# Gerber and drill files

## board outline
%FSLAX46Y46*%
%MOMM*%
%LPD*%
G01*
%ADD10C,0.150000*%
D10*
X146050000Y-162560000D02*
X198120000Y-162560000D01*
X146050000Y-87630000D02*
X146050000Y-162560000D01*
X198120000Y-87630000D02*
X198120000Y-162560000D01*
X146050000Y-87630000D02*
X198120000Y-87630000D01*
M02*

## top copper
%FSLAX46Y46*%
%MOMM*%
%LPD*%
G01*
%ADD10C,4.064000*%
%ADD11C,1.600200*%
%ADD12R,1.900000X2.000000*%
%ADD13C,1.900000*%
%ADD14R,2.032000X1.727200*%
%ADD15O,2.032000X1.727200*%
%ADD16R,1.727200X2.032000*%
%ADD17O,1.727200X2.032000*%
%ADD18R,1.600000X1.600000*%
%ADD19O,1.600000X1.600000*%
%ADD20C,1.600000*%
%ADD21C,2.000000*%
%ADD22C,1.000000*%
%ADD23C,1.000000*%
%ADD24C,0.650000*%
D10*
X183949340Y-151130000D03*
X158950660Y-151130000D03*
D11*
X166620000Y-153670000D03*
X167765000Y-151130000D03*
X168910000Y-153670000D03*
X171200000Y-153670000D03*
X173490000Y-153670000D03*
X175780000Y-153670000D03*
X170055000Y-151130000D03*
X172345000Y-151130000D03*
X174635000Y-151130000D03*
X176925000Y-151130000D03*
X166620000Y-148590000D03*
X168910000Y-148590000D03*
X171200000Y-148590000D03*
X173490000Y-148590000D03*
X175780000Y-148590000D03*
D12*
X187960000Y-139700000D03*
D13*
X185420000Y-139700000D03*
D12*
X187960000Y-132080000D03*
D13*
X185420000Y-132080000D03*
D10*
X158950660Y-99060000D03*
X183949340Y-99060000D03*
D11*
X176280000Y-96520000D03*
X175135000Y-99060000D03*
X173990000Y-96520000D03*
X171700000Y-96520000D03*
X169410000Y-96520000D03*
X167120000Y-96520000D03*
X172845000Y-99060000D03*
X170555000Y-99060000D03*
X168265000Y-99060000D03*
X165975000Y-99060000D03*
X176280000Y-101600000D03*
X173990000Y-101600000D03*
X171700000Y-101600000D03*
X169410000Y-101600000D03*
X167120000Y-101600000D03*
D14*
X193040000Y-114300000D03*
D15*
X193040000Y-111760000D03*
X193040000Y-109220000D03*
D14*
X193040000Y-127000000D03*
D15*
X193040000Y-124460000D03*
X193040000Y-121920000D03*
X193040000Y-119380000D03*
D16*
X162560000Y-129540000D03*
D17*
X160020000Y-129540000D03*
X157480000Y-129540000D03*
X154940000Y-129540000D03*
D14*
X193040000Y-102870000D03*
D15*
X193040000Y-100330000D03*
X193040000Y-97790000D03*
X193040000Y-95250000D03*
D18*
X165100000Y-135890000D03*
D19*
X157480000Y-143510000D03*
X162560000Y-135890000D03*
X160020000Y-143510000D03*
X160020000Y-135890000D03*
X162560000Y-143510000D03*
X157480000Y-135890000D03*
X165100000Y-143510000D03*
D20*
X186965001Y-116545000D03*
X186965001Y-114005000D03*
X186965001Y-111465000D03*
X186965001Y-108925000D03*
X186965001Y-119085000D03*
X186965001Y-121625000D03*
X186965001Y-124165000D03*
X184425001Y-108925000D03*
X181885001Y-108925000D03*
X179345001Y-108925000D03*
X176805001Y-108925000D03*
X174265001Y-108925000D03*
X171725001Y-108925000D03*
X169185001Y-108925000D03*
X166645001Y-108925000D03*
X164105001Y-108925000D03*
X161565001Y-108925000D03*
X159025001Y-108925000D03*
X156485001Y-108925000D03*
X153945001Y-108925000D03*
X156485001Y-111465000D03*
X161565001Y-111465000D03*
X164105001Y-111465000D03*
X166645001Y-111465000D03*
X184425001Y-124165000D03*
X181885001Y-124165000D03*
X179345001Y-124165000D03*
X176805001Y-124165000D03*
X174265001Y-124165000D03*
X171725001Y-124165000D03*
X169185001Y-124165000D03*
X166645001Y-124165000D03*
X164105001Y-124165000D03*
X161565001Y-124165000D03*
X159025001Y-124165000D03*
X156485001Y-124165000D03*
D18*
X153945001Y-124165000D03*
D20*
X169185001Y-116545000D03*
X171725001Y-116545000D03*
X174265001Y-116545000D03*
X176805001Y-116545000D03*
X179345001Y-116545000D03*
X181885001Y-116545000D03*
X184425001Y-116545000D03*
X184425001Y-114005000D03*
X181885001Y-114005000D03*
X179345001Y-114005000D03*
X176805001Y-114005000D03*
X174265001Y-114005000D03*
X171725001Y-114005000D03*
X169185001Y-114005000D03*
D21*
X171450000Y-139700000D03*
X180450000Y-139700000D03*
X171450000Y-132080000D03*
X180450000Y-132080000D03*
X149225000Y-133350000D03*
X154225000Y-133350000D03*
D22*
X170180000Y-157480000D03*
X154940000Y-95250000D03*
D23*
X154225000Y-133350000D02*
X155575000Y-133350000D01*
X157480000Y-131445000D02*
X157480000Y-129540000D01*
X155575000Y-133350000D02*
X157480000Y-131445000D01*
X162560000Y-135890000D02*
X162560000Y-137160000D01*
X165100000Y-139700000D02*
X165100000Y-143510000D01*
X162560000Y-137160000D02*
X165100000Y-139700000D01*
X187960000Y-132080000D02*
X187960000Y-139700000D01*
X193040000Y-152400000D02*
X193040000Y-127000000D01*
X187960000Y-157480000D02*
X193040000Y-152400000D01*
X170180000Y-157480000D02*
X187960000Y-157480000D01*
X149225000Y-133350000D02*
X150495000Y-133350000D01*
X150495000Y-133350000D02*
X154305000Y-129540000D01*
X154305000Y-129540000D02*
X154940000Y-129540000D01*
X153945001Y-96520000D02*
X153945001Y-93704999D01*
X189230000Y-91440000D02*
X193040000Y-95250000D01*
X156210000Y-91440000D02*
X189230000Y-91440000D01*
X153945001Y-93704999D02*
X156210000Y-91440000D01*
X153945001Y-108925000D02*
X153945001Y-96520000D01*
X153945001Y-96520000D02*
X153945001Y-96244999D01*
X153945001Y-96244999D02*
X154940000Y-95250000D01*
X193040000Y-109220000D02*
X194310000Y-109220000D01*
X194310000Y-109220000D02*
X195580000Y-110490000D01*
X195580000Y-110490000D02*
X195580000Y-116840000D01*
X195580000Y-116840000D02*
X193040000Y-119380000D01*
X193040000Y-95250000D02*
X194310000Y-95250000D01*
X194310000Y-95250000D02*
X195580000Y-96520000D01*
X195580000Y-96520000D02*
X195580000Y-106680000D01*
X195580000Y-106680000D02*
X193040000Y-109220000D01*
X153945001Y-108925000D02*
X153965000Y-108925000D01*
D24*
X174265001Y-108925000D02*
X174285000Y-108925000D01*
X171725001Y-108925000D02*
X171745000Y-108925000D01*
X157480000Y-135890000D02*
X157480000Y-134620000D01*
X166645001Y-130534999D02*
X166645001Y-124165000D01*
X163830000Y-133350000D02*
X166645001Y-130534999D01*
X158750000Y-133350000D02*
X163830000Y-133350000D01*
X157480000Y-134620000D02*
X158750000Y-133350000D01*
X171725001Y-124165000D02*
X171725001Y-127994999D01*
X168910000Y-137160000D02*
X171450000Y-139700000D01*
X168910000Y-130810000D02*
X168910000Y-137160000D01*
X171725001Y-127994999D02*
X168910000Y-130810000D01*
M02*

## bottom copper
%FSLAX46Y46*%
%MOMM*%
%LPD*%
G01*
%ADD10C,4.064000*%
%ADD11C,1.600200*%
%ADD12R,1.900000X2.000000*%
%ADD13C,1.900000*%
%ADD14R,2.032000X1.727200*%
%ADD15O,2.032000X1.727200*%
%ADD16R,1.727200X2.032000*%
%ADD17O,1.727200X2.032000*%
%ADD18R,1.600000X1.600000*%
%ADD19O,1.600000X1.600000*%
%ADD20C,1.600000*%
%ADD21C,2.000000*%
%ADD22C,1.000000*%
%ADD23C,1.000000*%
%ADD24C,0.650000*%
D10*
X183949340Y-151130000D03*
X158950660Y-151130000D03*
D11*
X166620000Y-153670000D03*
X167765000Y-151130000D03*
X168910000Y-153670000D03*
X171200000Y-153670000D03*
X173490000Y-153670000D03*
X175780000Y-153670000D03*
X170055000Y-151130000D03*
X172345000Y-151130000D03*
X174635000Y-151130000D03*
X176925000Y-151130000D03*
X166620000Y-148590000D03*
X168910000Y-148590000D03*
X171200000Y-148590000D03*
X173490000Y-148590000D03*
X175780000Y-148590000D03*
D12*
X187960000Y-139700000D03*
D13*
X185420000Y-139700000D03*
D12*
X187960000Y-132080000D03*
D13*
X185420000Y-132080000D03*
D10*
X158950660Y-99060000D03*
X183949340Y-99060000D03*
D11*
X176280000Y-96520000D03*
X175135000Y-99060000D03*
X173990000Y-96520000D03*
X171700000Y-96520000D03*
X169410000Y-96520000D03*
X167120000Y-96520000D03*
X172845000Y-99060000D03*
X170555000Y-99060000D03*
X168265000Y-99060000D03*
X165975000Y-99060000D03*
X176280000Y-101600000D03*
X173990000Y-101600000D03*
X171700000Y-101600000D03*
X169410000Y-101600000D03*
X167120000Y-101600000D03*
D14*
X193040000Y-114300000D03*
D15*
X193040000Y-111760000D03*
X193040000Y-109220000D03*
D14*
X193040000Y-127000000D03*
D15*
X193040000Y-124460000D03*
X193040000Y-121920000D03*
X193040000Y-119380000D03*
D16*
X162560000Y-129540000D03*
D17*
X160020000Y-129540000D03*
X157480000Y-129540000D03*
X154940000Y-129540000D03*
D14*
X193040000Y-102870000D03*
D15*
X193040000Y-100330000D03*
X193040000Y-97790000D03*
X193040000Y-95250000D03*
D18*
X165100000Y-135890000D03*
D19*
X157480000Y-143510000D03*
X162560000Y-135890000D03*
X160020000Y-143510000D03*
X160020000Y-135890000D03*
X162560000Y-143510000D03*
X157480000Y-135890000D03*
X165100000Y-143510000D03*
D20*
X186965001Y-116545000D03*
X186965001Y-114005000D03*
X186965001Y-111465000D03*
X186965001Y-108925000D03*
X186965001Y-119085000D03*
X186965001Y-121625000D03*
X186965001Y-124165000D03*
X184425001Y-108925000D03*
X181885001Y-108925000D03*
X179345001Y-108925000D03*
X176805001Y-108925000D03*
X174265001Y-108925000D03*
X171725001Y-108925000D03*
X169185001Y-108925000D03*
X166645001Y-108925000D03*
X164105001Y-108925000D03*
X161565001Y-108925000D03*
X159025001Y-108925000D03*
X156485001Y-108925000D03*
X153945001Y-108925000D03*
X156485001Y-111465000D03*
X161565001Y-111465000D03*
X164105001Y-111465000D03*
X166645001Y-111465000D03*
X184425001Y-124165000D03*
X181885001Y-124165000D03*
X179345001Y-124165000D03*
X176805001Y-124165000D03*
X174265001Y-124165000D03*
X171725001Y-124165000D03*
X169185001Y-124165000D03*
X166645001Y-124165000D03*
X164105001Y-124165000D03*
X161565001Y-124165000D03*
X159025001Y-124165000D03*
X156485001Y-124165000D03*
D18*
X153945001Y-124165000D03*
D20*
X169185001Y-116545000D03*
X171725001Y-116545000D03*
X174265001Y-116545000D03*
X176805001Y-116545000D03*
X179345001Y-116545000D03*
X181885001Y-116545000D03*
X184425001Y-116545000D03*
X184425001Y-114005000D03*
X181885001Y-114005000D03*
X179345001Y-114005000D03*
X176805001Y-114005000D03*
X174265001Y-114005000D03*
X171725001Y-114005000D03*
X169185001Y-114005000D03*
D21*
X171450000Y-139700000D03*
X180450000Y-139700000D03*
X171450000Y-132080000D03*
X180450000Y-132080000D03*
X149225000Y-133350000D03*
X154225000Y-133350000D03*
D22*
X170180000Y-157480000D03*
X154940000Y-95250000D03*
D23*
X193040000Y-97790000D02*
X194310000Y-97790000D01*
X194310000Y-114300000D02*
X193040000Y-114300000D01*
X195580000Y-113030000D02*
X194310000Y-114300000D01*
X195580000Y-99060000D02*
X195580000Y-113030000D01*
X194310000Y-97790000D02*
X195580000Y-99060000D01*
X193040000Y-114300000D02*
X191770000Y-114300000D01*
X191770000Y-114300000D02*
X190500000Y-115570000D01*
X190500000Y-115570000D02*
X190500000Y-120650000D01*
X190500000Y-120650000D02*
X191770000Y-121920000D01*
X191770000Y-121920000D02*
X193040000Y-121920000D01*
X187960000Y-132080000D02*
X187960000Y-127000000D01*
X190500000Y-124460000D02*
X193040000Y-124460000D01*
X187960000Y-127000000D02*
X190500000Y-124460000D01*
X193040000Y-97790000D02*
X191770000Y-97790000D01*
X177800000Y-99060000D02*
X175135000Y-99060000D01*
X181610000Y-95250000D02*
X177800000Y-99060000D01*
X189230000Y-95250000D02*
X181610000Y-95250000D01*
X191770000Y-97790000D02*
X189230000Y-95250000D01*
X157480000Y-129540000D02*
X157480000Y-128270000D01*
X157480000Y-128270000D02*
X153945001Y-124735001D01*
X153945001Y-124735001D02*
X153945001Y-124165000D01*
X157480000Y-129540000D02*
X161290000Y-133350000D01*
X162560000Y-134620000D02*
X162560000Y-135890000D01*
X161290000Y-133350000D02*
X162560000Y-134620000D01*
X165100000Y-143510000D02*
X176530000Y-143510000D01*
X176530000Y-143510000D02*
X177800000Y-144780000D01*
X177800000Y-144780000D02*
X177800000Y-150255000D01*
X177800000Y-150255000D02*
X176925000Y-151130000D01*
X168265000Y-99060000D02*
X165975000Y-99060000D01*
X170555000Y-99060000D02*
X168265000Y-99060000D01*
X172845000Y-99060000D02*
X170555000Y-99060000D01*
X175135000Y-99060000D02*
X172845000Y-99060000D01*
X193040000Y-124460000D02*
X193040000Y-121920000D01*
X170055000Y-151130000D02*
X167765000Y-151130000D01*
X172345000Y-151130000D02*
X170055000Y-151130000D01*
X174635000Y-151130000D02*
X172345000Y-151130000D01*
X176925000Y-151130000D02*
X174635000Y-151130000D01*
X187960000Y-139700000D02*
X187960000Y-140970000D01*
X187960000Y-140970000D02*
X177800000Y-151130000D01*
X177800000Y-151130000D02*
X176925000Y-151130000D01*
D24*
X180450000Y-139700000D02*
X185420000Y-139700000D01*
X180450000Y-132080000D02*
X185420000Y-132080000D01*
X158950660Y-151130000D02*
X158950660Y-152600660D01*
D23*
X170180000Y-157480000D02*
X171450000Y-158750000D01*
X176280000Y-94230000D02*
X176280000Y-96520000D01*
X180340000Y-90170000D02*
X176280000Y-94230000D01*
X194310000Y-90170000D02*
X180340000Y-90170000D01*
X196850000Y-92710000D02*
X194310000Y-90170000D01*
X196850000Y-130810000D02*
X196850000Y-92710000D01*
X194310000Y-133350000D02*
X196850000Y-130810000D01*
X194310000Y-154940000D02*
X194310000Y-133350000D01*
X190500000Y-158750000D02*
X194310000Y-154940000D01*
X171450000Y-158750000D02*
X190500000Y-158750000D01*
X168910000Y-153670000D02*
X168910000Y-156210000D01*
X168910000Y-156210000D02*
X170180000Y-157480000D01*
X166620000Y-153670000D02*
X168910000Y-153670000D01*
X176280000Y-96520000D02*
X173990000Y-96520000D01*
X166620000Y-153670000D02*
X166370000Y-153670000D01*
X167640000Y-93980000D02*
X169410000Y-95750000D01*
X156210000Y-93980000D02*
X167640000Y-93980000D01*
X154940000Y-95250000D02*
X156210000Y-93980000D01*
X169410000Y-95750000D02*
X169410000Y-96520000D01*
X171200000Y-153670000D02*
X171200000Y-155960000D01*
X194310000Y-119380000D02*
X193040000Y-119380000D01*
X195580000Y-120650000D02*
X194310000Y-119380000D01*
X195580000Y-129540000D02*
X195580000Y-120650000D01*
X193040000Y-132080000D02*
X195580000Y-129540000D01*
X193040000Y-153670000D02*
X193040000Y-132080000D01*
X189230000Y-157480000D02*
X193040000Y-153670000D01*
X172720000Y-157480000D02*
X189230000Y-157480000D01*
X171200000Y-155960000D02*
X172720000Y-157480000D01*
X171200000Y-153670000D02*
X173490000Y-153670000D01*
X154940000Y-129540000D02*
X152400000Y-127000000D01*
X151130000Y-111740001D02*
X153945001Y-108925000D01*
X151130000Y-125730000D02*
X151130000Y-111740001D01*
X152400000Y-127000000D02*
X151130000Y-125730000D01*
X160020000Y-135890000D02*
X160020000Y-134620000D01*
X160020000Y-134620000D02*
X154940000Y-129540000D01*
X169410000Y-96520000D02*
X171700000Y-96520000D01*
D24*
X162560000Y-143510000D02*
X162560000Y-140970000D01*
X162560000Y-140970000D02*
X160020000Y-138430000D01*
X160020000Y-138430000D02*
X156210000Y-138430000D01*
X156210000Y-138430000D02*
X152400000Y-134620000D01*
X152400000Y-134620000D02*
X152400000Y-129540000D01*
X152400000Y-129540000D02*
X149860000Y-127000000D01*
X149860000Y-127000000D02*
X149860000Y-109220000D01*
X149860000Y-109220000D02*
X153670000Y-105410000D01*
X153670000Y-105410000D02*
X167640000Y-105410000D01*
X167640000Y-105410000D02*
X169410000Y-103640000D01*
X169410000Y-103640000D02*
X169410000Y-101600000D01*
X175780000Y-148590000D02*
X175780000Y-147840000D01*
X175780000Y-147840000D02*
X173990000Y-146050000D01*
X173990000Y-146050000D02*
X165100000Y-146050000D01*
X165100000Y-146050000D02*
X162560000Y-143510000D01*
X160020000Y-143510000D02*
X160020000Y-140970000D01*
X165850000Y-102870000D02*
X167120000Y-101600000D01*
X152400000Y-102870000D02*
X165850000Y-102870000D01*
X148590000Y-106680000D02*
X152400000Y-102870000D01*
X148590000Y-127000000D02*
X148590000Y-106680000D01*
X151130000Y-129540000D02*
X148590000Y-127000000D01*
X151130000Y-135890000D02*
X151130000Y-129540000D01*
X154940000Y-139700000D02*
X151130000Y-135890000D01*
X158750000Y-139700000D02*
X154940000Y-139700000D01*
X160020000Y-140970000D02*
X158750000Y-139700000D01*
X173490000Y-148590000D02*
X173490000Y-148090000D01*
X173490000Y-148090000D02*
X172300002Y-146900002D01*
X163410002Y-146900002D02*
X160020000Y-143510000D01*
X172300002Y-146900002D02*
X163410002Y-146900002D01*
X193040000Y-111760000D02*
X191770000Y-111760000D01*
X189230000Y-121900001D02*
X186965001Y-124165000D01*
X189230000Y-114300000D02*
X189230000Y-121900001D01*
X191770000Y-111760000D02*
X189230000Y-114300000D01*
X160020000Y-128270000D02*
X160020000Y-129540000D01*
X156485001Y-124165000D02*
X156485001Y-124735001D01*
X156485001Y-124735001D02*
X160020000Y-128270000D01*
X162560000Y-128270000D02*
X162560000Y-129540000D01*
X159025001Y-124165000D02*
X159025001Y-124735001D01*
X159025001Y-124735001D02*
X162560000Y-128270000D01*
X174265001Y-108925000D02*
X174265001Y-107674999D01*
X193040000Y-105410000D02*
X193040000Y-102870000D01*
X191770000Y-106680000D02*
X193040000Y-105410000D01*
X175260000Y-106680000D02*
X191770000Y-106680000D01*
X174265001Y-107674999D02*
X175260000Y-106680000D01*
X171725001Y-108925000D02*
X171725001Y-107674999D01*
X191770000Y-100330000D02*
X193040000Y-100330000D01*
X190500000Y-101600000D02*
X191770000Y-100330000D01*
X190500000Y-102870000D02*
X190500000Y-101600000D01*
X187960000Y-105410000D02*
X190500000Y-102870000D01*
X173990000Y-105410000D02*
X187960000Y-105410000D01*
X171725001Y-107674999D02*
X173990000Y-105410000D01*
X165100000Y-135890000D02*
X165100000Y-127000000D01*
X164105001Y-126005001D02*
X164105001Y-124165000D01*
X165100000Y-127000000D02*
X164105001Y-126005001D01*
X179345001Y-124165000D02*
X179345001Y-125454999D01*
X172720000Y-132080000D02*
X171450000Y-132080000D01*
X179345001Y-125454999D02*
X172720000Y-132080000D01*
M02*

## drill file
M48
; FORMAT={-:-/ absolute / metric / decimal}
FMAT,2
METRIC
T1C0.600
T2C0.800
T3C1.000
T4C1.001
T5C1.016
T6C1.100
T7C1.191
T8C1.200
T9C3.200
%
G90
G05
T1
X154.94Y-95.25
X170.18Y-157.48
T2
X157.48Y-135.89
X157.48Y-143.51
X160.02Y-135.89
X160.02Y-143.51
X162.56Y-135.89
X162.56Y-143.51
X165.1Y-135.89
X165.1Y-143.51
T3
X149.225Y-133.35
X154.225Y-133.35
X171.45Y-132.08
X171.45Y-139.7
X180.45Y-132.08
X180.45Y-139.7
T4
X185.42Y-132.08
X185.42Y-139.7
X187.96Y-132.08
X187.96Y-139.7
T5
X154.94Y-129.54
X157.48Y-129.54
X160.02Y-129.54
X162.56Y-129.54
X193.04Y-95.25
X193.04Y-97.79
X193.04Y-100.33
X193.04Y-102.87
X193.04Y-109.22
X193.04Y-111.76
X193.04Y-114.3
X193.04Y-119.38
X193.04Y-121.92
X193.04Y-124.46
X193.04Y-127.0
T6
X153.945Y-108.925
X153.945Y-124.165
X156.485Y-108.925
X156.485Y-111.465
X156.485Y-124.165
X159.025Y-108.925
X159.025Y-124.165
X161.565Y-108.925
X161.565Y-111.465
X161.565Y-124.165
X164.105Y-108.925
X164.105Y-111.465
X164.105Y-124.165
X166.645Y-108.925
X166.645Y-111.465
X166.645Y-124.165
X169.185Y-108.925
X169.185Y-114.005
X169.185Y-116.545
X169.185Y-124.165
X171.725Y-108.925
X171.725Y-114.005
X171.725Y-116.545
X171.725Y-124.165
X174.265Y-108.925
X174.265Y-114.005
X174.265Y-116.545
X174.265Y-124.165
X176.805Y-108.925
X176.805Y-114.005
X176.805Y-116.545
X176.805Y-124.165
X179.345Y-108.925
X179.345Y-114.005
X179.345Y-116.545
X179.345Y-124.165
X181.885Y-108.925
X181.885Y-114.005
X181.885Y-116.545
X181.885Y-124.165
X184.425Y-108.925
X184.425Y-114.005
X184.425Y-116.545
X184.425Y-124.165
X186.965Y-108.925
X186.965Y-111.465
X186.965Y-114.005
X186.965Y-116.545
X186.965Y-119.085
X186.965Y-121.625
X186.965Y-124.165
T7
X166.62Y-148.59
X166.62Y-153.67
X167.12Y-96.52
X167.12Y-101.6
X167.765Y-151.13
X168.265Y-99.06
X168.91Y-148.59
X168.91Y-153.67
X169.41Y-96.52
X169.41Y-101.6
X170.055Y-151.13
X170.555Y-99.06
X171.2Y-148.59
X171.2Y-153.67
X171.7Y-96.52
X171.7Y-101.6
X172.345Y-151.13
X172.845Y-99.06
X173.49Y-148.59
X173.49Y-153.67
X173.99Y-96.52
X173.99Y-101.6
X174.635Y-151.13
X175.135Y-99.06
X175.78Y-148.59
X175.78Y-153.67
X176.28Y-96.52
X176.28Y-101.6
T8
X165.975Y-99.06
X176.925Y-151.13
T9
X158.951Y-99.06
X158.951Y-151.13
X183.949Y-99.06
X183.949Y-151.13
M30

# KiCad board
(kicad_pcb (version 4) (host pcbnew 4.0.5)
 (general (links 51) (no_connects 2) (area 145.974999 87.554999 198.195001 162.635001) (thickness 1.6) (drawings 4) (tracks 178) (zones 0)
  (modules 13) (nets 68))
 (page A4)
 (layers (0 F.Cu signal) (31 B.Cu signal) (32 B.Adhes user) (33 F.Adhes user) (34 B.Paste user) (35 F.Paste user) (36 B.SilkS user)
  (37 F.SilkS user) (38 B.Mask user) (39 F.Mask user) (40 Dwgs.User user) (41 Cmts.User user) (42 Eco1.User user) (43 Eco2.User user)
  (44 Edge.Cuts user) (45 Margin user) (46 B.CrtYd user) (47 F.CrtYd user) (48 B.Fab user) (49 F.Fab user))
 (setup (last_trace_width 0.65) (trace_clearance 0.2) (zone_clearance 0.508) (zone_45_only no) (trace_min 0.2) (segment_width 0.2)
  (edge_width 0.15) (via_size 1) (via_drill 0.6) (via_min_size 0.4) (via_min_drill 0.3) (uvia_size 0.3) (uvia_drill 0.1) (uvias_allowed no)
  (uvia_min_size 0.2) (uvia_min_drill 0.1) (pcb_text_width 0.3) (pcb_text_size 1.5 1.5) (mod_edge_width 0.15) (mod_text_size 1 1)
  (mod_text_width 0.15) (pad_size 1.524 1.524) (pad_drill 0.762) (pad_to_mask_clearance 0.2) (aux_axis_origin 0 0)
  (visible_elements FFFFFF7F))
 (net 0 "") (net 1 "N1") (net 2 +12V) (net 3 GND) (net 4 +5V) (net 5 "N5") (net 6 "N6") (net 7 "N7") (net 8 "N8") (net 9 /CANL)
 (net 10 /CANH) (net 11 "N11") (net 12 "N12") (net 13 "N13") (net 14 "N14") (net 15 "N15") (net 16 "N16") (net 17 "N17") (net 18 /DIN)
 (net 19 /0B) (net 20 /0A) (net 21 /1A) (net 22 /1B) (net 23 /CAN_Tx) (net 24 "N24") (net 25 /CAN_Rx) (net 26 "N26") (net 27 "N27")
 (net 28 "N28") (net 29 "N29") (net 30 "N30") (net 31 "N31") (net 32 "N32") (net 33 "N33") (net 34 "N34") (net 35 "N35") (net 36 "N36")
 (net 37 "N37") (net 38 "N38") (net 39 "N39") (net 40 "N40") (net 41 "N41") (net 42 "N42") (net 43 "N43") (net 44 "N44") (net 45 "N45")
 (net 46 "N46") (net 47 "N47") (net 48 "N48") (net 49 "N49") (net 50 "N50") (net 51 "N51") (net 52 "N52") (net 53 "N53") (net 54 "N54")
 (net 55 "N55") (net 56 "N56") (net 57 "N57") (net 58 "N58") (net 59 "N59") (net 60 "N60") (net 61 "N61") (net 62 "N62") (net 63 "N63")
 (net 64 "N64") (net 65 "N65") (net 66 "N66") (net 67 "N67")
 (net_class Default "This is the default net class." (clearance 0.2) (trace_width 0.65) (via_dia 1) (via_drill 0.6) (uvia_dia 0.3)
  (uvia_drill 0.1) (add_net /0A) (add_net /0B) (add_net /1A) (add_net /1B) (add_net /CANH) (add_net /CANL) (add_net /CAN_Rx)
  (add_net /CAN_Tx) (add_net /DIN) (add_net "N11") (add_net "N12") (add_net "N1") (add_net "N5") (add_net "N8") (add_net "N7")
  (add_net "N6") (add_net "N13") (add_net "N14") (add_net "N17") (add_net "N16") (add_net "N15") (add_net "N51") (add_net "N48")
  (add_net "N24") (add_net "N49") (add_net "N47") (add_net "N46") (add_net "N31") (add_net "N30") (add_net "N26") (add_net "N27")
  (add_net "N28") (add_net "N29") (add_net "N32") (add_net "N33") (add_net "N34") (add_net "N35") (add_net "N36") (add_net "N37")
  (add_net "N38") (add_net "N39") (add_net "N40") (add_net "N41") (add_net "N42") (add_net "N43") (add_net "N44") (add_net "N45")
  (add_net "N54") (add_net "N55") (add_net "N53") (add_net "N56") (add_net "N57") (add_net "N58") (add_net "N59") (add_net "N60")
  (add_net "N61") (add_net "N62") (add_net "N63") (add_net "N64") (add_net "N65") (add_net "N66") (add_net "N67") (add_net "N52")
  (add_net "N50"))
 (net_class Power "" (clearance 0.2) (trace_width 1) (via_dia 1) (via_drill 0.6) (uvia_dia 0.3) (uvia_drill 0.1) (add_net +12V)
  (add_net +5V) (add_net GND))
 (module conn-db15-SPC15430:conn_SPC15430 (layer F.Cu) (at 171.45 151.13 180)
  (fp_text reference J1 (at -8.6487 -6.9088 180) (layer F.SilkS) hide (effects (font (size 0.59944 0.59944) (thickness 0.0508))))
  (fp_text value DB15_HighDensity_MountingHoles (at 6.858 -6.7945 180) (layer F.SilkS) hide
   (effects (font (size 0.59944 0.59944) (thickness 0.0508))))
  (pad 0 thru_hole circle (at -12.49934 0 180) (size 4.064 4.064) (drill 3.2004) (layers *.Cu *.Mask) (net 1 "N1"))
  (pad 0 thru_hole circle (at 12.49934 0 180) (size 4.064 4.064) (drill 3.2004) (layers *.Cu *.Mask) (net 1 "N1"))
  (pad 15 thru_hole circle (at 4.83 -2.54 180) (size 1.6002 1.6002) (drill 1.19126) (layers *.Cu *.Mask) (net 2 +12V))
  (pad 10 thru_hole circle (at 3.685 0 180) (size 1.6002 1.6002) (drill 1.19126) (layers *.Cu *.Mask) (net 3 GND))
  (pad 14 thru_hole circle (at 2.54 -2.54 180) (size 1.6002 1.6002) (drill 1.19126) (layers *.Cu *.Mask) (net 2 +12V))
  (pad 13 thru_hole circle (at 0.25 -2.54 180) (size 1.6002 1.6002) (drill 1.19126) (layers *.Cu *.Mask) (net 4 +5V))
  (pad 12 thru_hole circle (at -2.04 -2.54 180) (size 1.6002 1.6002) (drill 1.19126) (layers *.Cu *.Mask) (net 4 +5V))
  (pad 11 thru_hole circle (at -4.33 -2.54 180) (size 1.6002 1.6002) (drill 1.19126) (layers *.Cu *.Mask) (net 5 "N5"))
  (pad 9 thru_hole circle (at 1.395 0 180) (size 1.6002 1.6002) (drill 1.19126) (layers *.Cu *.Mask) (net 3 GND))
  (pad 8 thru_hole circle (at -0.895 0 180) (size 1.6002 1.6002) (drill 1.19126) (layers *.Cu *.Mask) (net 3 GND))
  (pad 7 thru_hole circle (at -3.185 0 180) (size 1.6002 1.6002) (drill 1.19126) (layers *.Cu *.Mask) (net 3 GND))
  (pad 6 thru_hole circle (at -5.475 0 180) (size 1.6002 1.6002) (drill 1.2) (layers *.Cu *.Mask) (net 3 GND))
  (pad 5 thru_hole circle (at 4.83 2.54 180) (size 1.6002 1.6002) (drill 1.19126) (layers *.Cu *.Mask) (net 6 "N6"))
  (pad 4 thru_hole circle (at 2.54 2.54 180) (size 1.6002 1.6002) (drill 1.19126) (layers *.Cu *.Mask) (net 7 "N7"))
  (pad 3 thru_hole circle (at 0.25 2.54 180) (size 1.6002 1.6002) (drill 1.19126) (layers *.Cu *.Mask) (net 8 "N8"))
  (pad 2 thru_hole circle (at -2.04 2.54 180) (size 1.6002 1.6002) (drill 1.19126) (layers *.Cu *.Mask) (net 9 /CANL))
  (pad 1 thru_hole circle (at -4.33 2.54 180) (size 1.6002 1.6002) (drill 1.19126) (layers *.Cu *.Mask) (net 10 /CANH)))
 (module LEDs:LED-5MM (layer F.Cu) (at 187.96 139.7 180)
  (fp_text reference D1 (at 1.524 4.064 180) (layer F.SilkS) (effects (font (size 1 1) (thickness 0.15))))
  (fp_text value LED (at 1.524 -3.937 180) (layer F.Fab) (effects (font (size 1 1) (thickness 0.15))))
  (pad 1 thru_hole rect (at 0 0 270) (size 2 1.9) (drill 1.00076) (layers *.Cu *.Mask) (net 3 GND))
  (pad 2 thru_hole circle (at 2.54 0 180) (size 1.9 1.9) (drill 1.00076) (layers *.Cu *.Mask) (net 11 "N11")))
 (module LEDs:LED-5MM (layer F.Cu) (at 187.96 132.08 180)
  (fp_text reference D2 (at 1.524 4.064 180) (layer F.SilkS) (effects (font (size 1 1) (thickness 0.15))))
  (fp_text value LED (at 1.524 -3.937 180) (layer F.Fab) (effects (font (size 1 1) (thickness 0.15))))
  (pad 1 thru_hole rect (at 0 0 270) (size 2 1.9) (drill 1.00076) (layers *.Cu *.Mask) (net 3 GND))
  (pad 2 thru_hole circle (at 2.54 0 180) (size 1.9 1.9) (drill 1.00076) (layers *.Cu *.Mask) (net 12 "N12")))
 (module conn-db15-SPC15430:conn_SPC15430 (layer F.Cu) (at 171.45 99.06)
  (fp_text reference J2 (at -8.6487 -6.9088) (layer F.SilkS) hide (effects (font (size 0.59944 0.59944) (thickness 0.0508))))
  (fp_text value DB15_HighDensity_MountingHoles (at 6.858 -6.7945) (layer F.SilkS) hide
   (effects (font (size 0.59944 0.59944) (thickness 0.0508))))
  (pad 0 thru_hole circle (at -12.49934 0) (size 4.064 4.064) (drill 3.2004) (layers *.Cu *.Mask) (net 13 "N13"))
  (pad 0 thru_hole circle (at 12.49934 0) (size 4.064 4.064) (drill 3.2004) (layers *.Cu *.Mask) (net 13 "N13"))
  (pad 15 thru_hole circle (at 4.83 -2.54) (size 1.6002 1.6002) (drill 1.19126) (layers *.Cu *.Mask) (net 2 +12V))
  (pad 10 thru_hole circle (at 3.685 0) (size 1.6002 1.6002) (drill 1.19126) (layers *.Cu *.Mask) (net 3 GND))
  (pad 14 thru_hole circle (at 2.54 -2.54) (size 1.6002 1.6002) (drill 1.19126) (layers *.Cu *.Mask) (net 2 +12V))
  (pad 13 thru_hole circle (at 0.25 -2.54) (size 1.6002 1.6002) (drill 1.19126) (layers *.Cu *.Mask) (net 4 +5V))
  (pad 12 thru_hole circle (at -2.04 -2.54) (size 1.6002 1.6002) (drill 1.19126) (layers *.Cu *.Mask) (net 4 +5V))
  (pad 11 thru_hole circle (at -4.33 -2.54) (size 1.6002 1.6002) (drill 1.19126) (layers *.Cu *.Mask) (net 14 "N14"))
  (pad 9 thru_hole circle (at 1.395 0) (size 1.6002 1.6002) (drill 1.19126) (layers *.Cu *.Mask) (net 3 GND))
  (pad 8 thru_hole circle (at -0.895 0) (size 1.6002 1.6002) (drill 1.19126) (layers *.Cu *.Mask) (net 3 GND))
  (pad 7 thru_hole circle (at -3.185 0) (size 1.6002 1.6002) (drill 1.19126) (layers *.Cu *.Mask) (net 3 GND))
  (pad 6 thru_hole circle (at -5.475 0) (size 1.6002 1.6002) (drill 1.2) (layers *.Cu *.Mask) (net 3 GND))
  (pad 5 thru_hole circle (at 4.83 2.54) (size 1.6002 1.6002) (drill 1.19126) (layers *.Cu *.Mask) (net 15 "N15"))
  (pad 4 thru_hole circle (at 2.54 2.54) (size 1.6002 1.6002) (drill 1.19126) (layers *.Cu *.Mask) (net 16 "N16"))
  (pad 3 thru_hole circle (at 0.25 2.54) (size 1.6002 1.6002) (drill 1.19126) (layers *.Cu *.Mask) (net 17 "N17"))
  (pad 2 thru_hole circle (at -2.04 2.54) (size 1.6002 1.6002) (drill 1.19126) (layers *.Cu *.Mask) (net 10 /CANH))
  (pad 1 thru_hole circle (at -4.33 2.54) (size 1.6002 1.6002) (drill 1.19126) (layers *.Cu *.Mask) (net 9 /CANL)))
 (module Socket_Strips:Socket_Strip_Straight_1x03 (layer F.Cu) (at 193.04 114.3 90)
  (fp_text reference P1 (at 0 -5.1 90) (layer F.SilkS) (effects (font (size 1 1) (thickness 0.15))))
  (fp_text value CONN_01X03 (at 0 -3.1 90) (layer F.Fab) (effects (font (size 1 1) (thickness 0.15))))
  (pad 1 thru_hole rect (at 0 0 90) (size 1.7272 2.032) (drill 1.016) (layers *.Cu *.Mask) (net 3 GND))
  (pad 2 thru_hole oval (at 2.54 0 90) (size 1.7272 2.032) (drill 1.016) (layers *.Cu *.Mask) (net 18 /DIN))
  (pad 3 thru_hole oval (at 5.08 0 90) (size 1.7272 2.032) (drill 1.016) (layers *.Cu *.Mask) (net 4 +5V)))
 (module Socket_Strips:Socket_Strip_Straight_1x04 (layer F.Cu) (at 193.04 127 90)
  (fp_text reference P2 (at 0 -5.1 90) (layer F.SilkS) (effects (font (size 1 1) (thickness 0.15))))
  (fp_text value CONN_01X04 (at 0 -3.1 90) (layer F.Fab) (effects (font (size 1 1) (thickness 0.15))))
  (pad 1 thru_hole rect (at 0 0 90) (size 1.7272 2.032) (drill 1.016) (layers *.Cu *.Mask) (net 2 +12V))
  (pad 2 thru_hole oval (at 2.54 0 90) (size 1.7272 2.032) (drill 1.016) (layers *.Cu *.Mask) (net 3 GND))
  (pad 3 thru_hole oval (at 5.08 0 90) (size 1.7272 2.032) (drill 1.016) (layers *.Cu *.Mask) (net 3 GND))
  (pad 4 thru_hole oval (at 7.62 0 90) (size 1.7272 2.032) (drill 1.016) (layers *.Cu *.Mask) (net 4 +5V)))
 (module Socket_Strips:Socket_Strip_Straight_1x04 (layer F.Cu) (at 162.56 129.54 180)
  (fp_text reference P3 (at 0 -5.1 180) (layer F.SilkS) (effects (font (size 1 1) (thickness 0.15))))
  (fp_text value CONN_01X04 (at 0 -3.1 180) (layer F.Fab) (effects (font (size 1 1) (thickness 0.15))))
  (pad 1 thru_hole rect (at 0 0 180) (size 1.7272 2.032) (drill 1.016) (layers *.Cu *.Mask) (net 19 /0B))
  (pad 2 thru_hole oval (at 2.54 0 180) (size 1.7272 2.032) (drill 1.016) (layers *.Cu *.Mask) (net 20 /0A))
  (pad 3 thru_hole oval (at 5.08 0 180) (size 1.7272 2.032) (drill 1.016) (layers *.Cu *.Mask) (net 3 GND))
  (pad 4 thru_hole oval (at 7.62 0 180) (size 1.7272 2.032) (drill 1.016) (layers *.Cu *.Mask) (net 4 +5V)))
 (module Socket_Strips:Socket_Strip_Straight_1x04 (layer F.Cu) (at 193.04 102.87 90)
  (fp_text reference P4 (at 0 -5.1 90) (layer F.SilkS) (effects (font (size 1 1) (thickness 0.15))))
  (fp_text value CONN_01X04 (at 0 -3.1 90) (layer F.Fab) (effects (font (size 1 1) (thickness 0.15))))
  (pad 1 thru_hole rect (at 0 0 90) (size 1.7272 2.032) (drill 1.016) (layers *.Cu *.Mask) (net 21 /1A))
  (pad 2 thru_hole oval (at 2.54 0 90) (size 1.7272 2.032) (drill 1.016) (layers *.Cu *.Mask) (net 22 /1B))
  (pad 3 thru_hole oval (at 5.08 0 90) (size 1.7272 2.032) (drill 1.016) (layers *.Cu *.Mask) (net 3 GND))
  (pad 4 thru_hole oval (at 7.62 0 90) (size 1.7272 2.032) (drill 1.016) (layers *.Cu *.Mask) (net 4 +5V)))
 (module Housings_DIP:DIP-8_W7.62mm (layer F.Cu) (at 165.1 135.89 270)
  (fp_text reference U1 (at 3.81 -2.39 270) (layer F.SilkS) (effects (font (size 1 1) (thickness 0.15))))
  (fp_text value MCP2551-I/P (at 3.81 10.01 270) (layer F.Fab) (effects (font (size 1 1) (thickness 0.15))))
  (pad 1 thru_hole rect (at 0 0 270) (size 1.6 1.6) (drill 0.8) (layers *.Cu *.Mask) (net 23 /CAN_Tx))
  (pad 5 thru_hole oval (at 7.62 7.62 270) (size 1.6 1.6) (drill 0.8) (layers *.Cu *.Mask) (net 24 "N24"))
  (pad 2 thru_hole oval (at 0 2.54 270) (size 1.6 1.6) (drill 0.8) (layers *.Cu *.Mask) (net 3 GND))
  (pad 6 thru_hole oval (at 7.62 5.08 270) (size 1.6 1.6) (drill 0.8) (layers *.Cu *.Mask) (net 9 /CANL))
  (pad 3 thru_hole oval (at 0 5.08 270) (size 1.6 1.6) (drill 0.8) (layers *.Cu *.Mask) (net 4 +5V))
  (pad 7 thru_hole oval (at 7.62 2.54 270) (size 1.6 1.6) (drill 0.8) (layers *.Cu *.Mask) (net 10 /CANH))
  (pad 4 thru_hole oval (at 0 7.62 270) (size 1.6 1.6) (drill 0.8) (layers *.Cu *.Mask) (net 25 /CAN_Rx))
  (pad 8 thru_hole oval (at 7.62 0 270) (size 1.6 1.6) (drill 0.8) (layers *.Cu *.Mask) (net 3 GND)))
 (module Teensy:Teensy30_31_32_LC (layer F.Cu) (at 170.455001 116.545)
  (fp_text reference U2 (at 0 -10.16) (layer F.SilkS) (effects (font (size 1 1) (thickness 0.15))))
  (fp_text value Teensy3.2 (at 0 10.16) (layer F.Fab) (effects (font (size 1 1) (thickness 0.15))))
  (pad 17 thru_hole circle (at 16.51 0) (size 1.6 1.6) (drill 1.1) (layers *.Cu *.Mask F.SilkS) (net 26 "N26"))
  (pad 18 thru_hole circle (at 16.51 -2.54) (size 1.6 1.6) (drill 1.1) (layers *.Cu *.Mask F.SilkS) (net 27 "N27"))
  (pad 19 thru_hole circle (at 16.51 -5.08) (size 1.6 1.6) (drill 1.1) (layers *.Cu *.Mask F.SilkS) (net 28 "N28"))
  (pad 20 thru_hole circle (at 16.51 -7.62) (size 1.6 1.6) (drill 1.1) (layers *.Cu *.Mask F.SilkS) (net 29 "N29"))
  (pad 16 thru_hole circle (at 16.51 2.54) (size 1.6 1.6) (drill 1.1) (layers *.Cu *.Mask F.SilkS) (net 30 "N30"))
  (pad 15 thru_hole circle (at 16.51 5.08) (size 1.6 1.6) (drill 1.1) (layers *.Cu *.Mask F.SilkS) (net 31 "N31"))
  (pad 14 thru_hole circle (at 16.51 7.62) (size 1.6 1.6) (drill 1.1) (layers *.Cu *.Mask F.SilkS) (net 18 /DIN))
  (pad 21 thru_hole circle (at 13.97 -7.62) (size 1.6 1.6) (drill 1.1) (layers *.Cu *.Mask F.SilkS) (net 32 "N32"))
  (pad 22 thru_hole circle (at 11.43 -7.62) (size 1.6 1.6) (drill 1.1) (layers *.Cu *.Mask F.SilkS) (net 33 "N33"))
  (pad 23 thru_hole circle (at 8.89 -7.62) (size 1.6 1.6) (drill 1.1) (layers *.Cu *.Mask F.SilkS) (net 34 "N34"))
  (pad 24 thru_hole circle (at 6.35 -7.62) (size 1.6 1.6) (drill 1.1) (layers *.Cu *.Mask F.SilkS) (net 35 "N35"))
  (pad 25 thru_hole circle (at 3.81 -7.62) (size 1.6 1.6) (drill 1.1) (layers *.Cu *.Mask F.SilkS) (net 21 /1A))
  (pad 26 thru_hole circle (at 1.27 -7.62) (size 1.6 1.6) (drill 1.1) (layers *.Cu *.Mask F.SilkS) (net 22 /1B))
  (pad 27 thru_hole circle (at -1.27 -7.62) (size 1.6 1.6) (drill 1.1) (layers *.Cu *.Mask F.SilkS) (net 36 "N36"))
  (pad 28 thru_hole circle (at -3.81 -7.62) (size 1.6 1.6) (drill 1.1) (layers *.Cu *.Mask F.SilkS) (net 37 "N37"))
  (pad 29 thru_hole circle (at -6.35 -7.62) (size 1.6 1.6) (drill 1.1) (layers *.Cu *.Mask F.SilkS) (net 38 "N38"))
  (pad 30 thru_hole circle (at -8.89 -7.62) (size 1.6 1.6) (drill 1.1) (layers *.Cu *.Mask F.SilkS) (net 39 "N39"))
  (pad 31 thru_hole circle (at -11.43 -7.62) (size 1.6 1.6) (drill 1.1) (layers *.Cu *.Mask F.SilkS) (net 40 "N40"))
  (pad 32 thru_hole circle (at -13.97 -7.62) (size 1.6 1.6) (drill 1.1) (layers *.Cu *.Mask F.SilkS) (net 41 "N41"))
  (pad 33 thru_hole circle (at -16.51 -7.62) (size 1.6 1.6) (drill 1.1) (layers *.Cu *.Mask F.SilkS) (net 4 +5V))
  (pad 34 thru_hole circle (at -13.97 -5.08) (size 1.6 1.6) (drill 1.1) (layers *.Cu *.Mask F.SilkS) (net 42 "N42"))
  (pad 35 thru_hole circle (at -8.89 -5.08) (size 1.6 1.6) (drill 1.1) (layers *.Cu *.Mask F.SilkS) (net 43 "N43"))
  (pad 36 thru_hole circle (at -6.35 -5.08) (size 1.6 1.6) (drill 1.1) (layers *.Cu *.Mask F.SilkS) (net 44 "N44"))
  (pad 37 thru_hole circle (at -3.81 -5.08) (size 1.6 1.6) (drill 1.1) (layers *.Cu *.Mask F.SilkS) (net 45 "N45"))
  (pad 13 thru_hole circle (at 13.97 7.62) (size 1.6 1.6) (drill 1.1) (layers *.Cu *.Mask F.SilkS) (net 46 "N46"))
  (pad 12 thru_hole circle (at 11.43 7.62) (size 1.6 1.6) (drill 1.1) (layers *.Cu *.Mask F.SilkS) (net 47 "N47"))
  (pad 11 thru_hole circle (at 8.89 7.62) (size 1.6 1.6) (drill 1.1) (layers *.Cu *.Mask F.SilkS) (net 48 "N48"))
  (pad 10 thru_hole circle (at 6.35 7.62) (size 1.6 1.6) (drill 1.1) (layers *.Cu *.Mask F.SilkS) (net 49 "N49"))
  (pad 9 thru_hole circle (at 3.81 7.62) (size 1.6 1.6) (drill 1.1) (layers *.Cu *.Mask F.SilkS) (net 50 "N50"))
  (pad 8 thru_hole circle (at 1.27 7.62) (size 1.6 1.6) (drill 1.1) (layers *.Cu *.Mask F.SilkS) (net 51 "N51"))
  (pad 7 thru_hole circle (at -1.27 7.62) (size 1.6 1.6) (drill 1.1) (layers *.Cu *.Mask F.SilkS) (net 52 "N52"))
  (pad 6 thru_hole circle (at -3.81 7.62) (size 1.6 1.6) (drill 1.1) (layers *.Cu *.Mask F.SilkS) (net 25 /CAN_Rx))
  (pad 5 thru_hole circle (at -6.35 7.62) (size 1.6 1.6) (drill 1.1) (layers *.Cu *.Mask F.SilkS) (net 23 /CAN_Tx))
  (pad 4 thru_hole circle (at -8.89 7.62) (size 1.6 1.6) (drill 1.1) (layers *.Cu *.Mask F.SilkS) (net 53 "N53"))
  (pad 3 thru_hole circle (at -11.43 7.62) (size 1.6 1.6) (drill 1.1) (layers *.Cu *.Mask F.SilkS) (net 19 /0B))
  (pad 2 thru_hole circle (at -13.97 7.62) (size 1.6 1.6) (drill 1.1) (layers *.Cu *.Mask F.SilkS) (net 20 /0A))
  (pad 1 thru_hole rect (at -16.51 7.62) (size 1.6 1.6) (drill 1.1) (layers *.Cu *.Mask F.SilkS) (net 3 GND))
  (pad 38 thru_hole circle (at -1.27 0) (size 1.6 1.6) (drill 1.1) (layers *.Cu *.Mask) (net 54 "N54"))
  (pad 39 thru_hole circle (at 1.27 0) (size 1.6 1.6) (drill 1.1) (layers *.Cu *.Mask) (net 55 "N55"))
  (pad 40 thru_hole circle (at 3.81 0) (size 1.6 1.6) (drill 1.1) (layers *.Cu *.Mask) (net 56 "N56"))
  (pad 41 thru_hole circle (at 6.35 0) (size 1.6 1.6) (drill 1.1) (layers *.Cu *.Mask) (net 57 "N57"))
  (pad 42 thru_hole circle (at 8.89 0) (size 1.6 1.6) (drill 1.1) (layers *.Cu *.Mask) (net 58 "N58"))
  (pad 43 thru_hole circle (at 11.43 0) (size 1.6 1.6) (drill 1.1) (layers *.Cu *.Mask) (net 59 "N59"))
  (pad 44 thru_hole circle (at 13.97 0) (size 1.6 1.6) (drill 1.1) (layers *.Cu *.Mask) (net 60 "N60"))
  (pad 45 thru_hole circle (at 13.97 -2.54) (size 1.6 1.6) (drill 1.1) (layers *.Cu *.Mask) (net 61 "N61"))
  (pad 46 thru_hole circle (at 11.43 -2.54) (size 1.6 1.6) (drill 1.1) (layers *.Cu *.Mask) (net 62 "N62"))
  (pad 47 thru_hole circle (at 8.89 -2.54) (size 1.6 1.6) (drill 1.1) (layers *.Cu *.Mask) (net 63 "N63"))
  (pad 48 thru_hole circle (at 6.35 -2.54) (size 1.6 1.6) (drill 1.1) (layers *.Cu *.Mask) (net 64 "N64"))
  (pad 49 thru_hole circle (at 3.81 -2.54) (size 1.6 1.6) (drill 1.1) (layers *.Cu *.Mask) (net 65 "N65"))
  (pad 50 thru_hole circle (at 1.27 -2.54) (size 1.6 1.6) (drill 1.1) (layers *.Cu *.Mask) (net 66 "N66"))
  (pad 51 thru_hole circle (at -1.27 -2.54) (size 1.6 1.6) (drill 1.1) (layers *.Cu *.Mask) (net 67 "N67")))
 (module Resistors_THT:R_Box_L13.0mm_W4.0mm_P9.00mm (layer F.Cu) (at 171.45 139.7)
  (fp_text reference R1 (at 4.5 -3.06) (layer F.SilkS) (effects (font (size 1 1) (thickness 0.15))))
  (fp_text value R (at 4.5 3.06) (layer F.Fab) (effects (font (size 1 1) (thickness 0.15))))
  (pad 1 thru_hole circle (at 0 0) (size 2 2) (drill 1) (layers *.Cu *.Mask) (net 51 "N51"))
  (pad 2 thru_hole circle (at 9 0) (size 2 2) (drill 1) (layers *.Cu *.Mask) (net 11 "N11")))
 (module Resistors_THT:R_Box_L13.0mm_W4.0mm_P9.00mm (layer F.Cu) (at 171.45 132.08)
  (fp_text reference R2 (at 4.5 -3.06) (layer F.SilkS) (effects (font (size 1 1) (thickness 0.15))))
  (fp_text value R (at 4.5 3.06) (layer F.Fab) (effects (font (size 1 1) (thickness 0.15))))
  (pad 1 thru_hole circle (at 0 0) (size 2 2) (drill 1) (layers *.Cu *.Mask) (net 48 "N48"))
  (pad 2 thru_hole circle (at 9 0) (size 2 2) (drill 1) (layers *.Cu *.Mask) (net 12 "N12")))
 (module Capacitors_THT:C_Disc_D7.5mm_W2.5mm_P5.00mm (layer F.Cu) (at 149.225 133.35)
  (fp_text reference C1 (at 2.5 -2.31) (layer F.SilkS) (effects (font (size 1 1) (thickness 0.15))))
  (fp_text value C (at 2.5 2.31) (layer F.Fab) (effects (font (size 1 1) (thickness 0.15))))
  (pad 1 thru_hole circle (at 0 0) (size 2 2) (drill 1) (layers *.Cu *.Mask) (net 4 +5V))
  (pad 2 thru_hole circle (at 5 0) (size 2 2) (drill 1) (layers *.Cu *.Mask) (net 3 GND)))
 (gr_line (start 146.05 162.56) (end 198.12 162.56) (angle 90) (layer Edge.Cuts) (width 0.15))
 (gr_line (start 146.05 87.63) (end 146.05 162.56) (angle 90) (layer Edge.Cuts) (width 0.15))
 (gr_line (start 198.12 87.63) (end 198.12 162.56) (angle 90) (layer Edge.Cuts) (width 0.15))
 (gr_line (start 146.05 87.63) (end 198.12 87.63) (angle 90) (layer Edge.Cuts) (width 0.15))
 (segment (start 154.225 133.35) (end 155.575 133.35) (width 1) (layer F.Cu) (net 3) (status 400000))
 (segment (start 157.48 131.445) (end 157.48 129.54) (width 1) (layer F.Cu) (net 3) (status 800000))
 (segment (start 155.575 133.35) (end 157.48 131.445) (width 1) (layer F.Cu) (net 3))
 (segment (start 193.04 97.79) (end 194.31 97.79) (width 1) (layer B.Cu) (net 3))
 (segment (start 194.31 114.3) (end 193.04 114.3) (width 1) (layer B.Cu) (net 3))
 (segment (start 195.58 113.03) (end 194.31 114.3) (width 1) (layer B.Cu) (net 3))
 (segment (start 195.58 99.06) (end 195.58 113.03) (width 1) (layer B.Cu) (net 3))
 (segment (start 194.31 97.79) (end 195.58 99.06) (width 1) (layer B.Cu) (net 3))
 (segment (start 193.04 114.3) (end 191.77 114.3) (width 1) (layer B.Cu) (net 3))
 (segment (start 191.77 114.3) (end 190.5 115.57) (width 1) (layer B.Cu) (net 3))
 (segment (start 190.5 115.57) (end 190.5 120.65) (width 1) (layer B.Cu) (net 3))
 (segment (start 190.5 120.65) (end 191.77 121.92) (width 1) (layer B.Cu) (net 3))
 (segment (start 191.77 121.92) (end 193.04 121.92) (width 1) (layer B.Cu) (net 3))
 (segment (start 187.96 132.08) (end 187.96 127) (width 1) (layer B.Cu) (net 3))
 (segment (start 190.5 124.46) (end 193.04 124.46) (width 1) (layer B.Cu) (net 3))
 (segment (start 187.96 127) (end 190.5 124.46) (width 1) (layer B.Cu) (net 3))
 (segment (start 193.04 97.79) (end 191.77 97.79) (width 1) (layer B.Cu) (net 3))
 (segment (start 177.8 99.06) (end 175.135 99.06) (width 1) (layer B.Cu) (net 3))
 (segment (start 181.61 95.25) (end 177.8 99.06) (width 1) (layer B.Cu) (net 3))
 (segment (start 189.23 95.25) (end 181.61 95.25) (width 1) (layer B.Cu) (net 3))
 (segment (start 191.77 97.79) (end 189.23 95.25) (width 1) (layer B.Cu) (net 3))
 (segment (start 162.56 135.89) (end 162.56 137.16) (width 1) (layer F.Cu) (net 3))
 (segment (start 165.1 139.7) (end 165.1 143.51) (width 1) (layer F.Cu) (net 3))
 (segment (start 162.56 137.16) (end 165.1 139.7) (width 1) (layer F.Cu) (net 3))
 (segment (start 187.96 132.08) (end 187.96 139.7) (width 1) (layer F.Cu) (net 3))
 (segment (start 157.48 129.54) (end 157.48 128.27) (width 1) (layer B.Cu) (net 3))
 (segment (start 157.48 128.27) (end 153.945001 124.735001) (width 1) (layer B.Cu) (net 3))
 (segment (start 153.945001 124.735001) (end 153.945001 124.165) (width 1) (layer B.Cu) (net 3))
 (segment (start 157.48 129.54) (end 161.29 133.35) (width 1) (layer B.Cu) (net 3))
 (segment (start 162.56 134.62) (end 162.56 135.89) (width 1) (layer B.Cu) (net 3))
 (segment (start 161.29 133.35) (end 162.56 134.62) (width 1) (layer B.Cu) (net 3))
 (segment (start 165.1 143.51) (end 176.53 143.51) (width 1) (layer B.Cu) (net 3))
 (segment (start 176.53 143.51) (end 177.8 144.78) (width 1) (layer B.Cu) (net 3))
 (segment (start 177.8 144.78) (end 177.8 150.255) (width 1) (layer B.Cu) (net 3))
 (segment (start 177.8 150.255) (end 176.925 151.13) (width 1) (layer B.Cu) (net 3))
 (segment (start 168.265 99.06) (end 165.975 99.06) (width 1) (layer B.Cu) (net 3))
 (segment (start 170.555 99.06) (end 168.265 99.06) (width 1) (layer B.Cu) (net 3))
 (segment (start 172.845 99.06) (end 170.555 99.06) (width 1) (layer B.Cu) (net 3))
 (segment (start 175.135 99.06) (end 172.845 99.06) (width 1) (layer B.Cu) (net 3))
 (segment (start 193.04 124.46) (end 193.04 121.92) (width 1) (layer B.Cu) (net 3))
 (segment (start 170.055 151.13) (end 167.765 151.13) (width 1) (layer B.Cu) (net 3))
 (segment (start 172.345 151.13) (end 170.055 151.13) (width 1) (layer B.Cu) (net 3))
 (segment (start 174.635 151.13) (end 172.345 151.13) (width 1) (layer B.Cu) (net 3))
 (segment (start 176.925 151.13) (end 174.635 151.13) (width 1) (layer B.Cu) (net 3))
 (segment (start 187.96 139.7) (end 187.96 140.97) (width 1) (layer B.Cu) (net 3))
 (segment (start 187.96 140.97) (end 177.8 151.13) (width 1) (layer B.Cu) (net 3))
 (segment (start 177.8 151.13) (end 176.925 151.13) (width 1) (layer B.Cu) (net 3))
 (segment (start 180.45 139.7) (end 185.42 139.7) (width 0.65) (layer B.Cu) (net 11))
 (segment (start 180.45 132.08) (end 185.42 132.08) (width 0.65) (layer B.Cu) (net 12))
 (segment (start 158.95066 151.13) (end 158.95066 152.60066) (width 0.65) (layer B.Cu) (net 1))
 (segment (start 170.18 157.48) (end 171.45 158.75) (width 1) (layer B.Cu) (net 2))
 (segment (start 176.28 94.23) (end 176.28 96.52) (width 1) (layer B.Cu) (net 2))
 (segment (start 180.34 90.17) (end 176.28 94.23) (width 1) (layer B.Cu) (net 2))
 (segment (start 194.31 90.17) (end 180.34 90.17) (width 1) (layer B.Cu) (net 2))
 (segment (start 196.85 92.71) (end 194.31 90.17) (width 1) (layer B.Cu) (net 2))
 (segment (start 196.85 130.81) (end 196.85 92.71) (width 1) (layer B.Cu) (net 2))
 (segment (start 194.31 133.35) (end 196.85 130.81) (width 1) (layer B.Cu) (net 2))
 (segment (start 194.31 154.94) (end 194.31 133.35) (width 1) (layer B.Cu) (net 2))
 (segment (start 190.5 158.75) (end 194.31 154.94) (width 1) (layer B.Cu) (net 2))
 (segment (start 171.45 158.75) (end 190.5 158.75) (width 1) (layer B.Cu) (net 2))
 (segment (start 168.91 153.67) (end 168.91 156.21) (width 1) (layer B.Cu) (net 2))
 (segment (start 193.04 152.4) (end 193.04 127) (width 1) (layer F.Cu) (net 2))
 (segment (start 187.96 157.48) (end 193.04 152.4) (width 1) (layer F.Cu) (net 2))
 (segment (start 170.18 157.48) (end 187.96 157.48) (width 1) (layer F.Cu) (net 2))
 (via (at 170.18 157.48) (size 1) (drill 0.6) (layers F.Cu B.Cu) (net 2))
 (segment (start 168.91 156.21) (end 170.18 157.48) (width 1) (layer B.Cu) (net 2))
 (segment (start 166.62 153.67) (end 168.91 153.67) (width 1) (layer B.Cu) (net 2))
 (segment (start 176.28 96.52) (end 173.99 96.52) (width 1) (layer B.Cu) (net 2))
 (segment (start 166.62 153.67) (end 166.37 153.67) (width 1) (layer B.Cu) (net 2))
 (segment (start 149.225 133.35) (end 150.495 133.35) (width 1) (layer F.Cu) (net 4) (status 400000))
 (segment (start 150.495 133.35) (end 154.305 129.54) (width 1) (layer F.Cu) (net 4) (status 800000))
 (segment (start 154.305 129.54) (end 154.94 129.54) (width 1) (layer F.Cu) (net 4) (status C00000))
 (segment (start 153.945001 96.52) (end 153.945001 93.704999) (width 1) (layer F.Cu) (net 4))
 (segment (start 189.23 91.44) (end 193.04 95.25) (width 1) (layer F.Cu) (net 4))
 (segment (start 156.21 91.44) (end 189.23 91.44) (width 1) (layer F.Cu) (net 4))
 (segment (start 153.945001 93.704999) (end 156.21 91.44) (width 1) (layer F.Cu) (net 4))
 (segment (start 153.945001 108.925) (end 153.945001 96.52) (width 1) (layer F.Cu) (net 4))
 (segment (start 153.945001 96.52) (end 153.945001 96.244999) (width 1) (layer F.Cu) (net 4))
 (segment (start 167.64 93.98) (end 169.41 95.75) (width 1) (layer B.Cu) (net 4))
 (segment (start 156.21 93.98) (end 167.64 93.98) (width 1) (layer B.Cu) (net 4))
 (segment (start 154.94 95.25) (end 156.21 93.98) (width 1) (layer B.Cu) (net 4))
 (via (at 154.94 95.25) (size 1) (drill 0.6) (layers F.Cu B.Cu) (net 4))
 (segment (start 153.945001 96.244999) (end 154.94 95.25) (width 1) (layer F.Cu) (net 4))
 (segment (start 169.41 95.75) (end 169.41 96.52) (width 1) (layer B.Cu) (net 4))
 (segment (start 171.2 153.67) (end 171.2 155.96) (width 1) (layer B.Cu) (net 4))
 (segment (start 194.31 119.38) (end 193.04 119.38) (width 1) (layer B.Cu) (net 4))
 (segment (start 195.58 120.65) (end 194.31 119.38) (width 1) (layer B.Cu) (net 4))
 (segment (start 195.58 129.54) (end 195.58 120.65) (width 1) (layer B.Cu) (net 4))
 (segment (start 193.04 132.08) (end 195.58 129.54) (width 1) (layer B.Cu) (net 4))
 (segment (start 193.04 153.67) (end 193.04 132.08) (width 1) (layer B.Cu) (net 4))
 (segment (start 189.23 157.48) (end 193.04 153.67) (width 1) (layer B.Cu) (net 4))
 (segment (start 172.72 157.48) (end 189.23 157.48) (width 1) (layer B.Cu) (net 4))
 (segment (start 171.2 155.96) (end 172.72 157.48) (width 1) (layer B.Cu) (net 4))
 (segment (start 193.04 109.22) (end 194.31 109.22) (width 1) (layer F.Cu) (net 4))
 (segment (start 194.31 109.22) (end 195.58 110.49) (width 1) (layer F.Cu) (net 4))
 (segment (start 195.58 110.49) (end 195.58 116.84) (width 1) (layer F.Cu) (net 4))
 (segment (start 195.58 116.84) (end 193.04 119.38) (width 1) (layer F.Cu) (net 4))
 (segment (start 193.04 95.25) (end 194.31 95.25) (width 1) (layer F.Cu) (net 4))
 (segment (start 194.31 95.25) (end 195.58 96.52) (width 1) (layer F.Cu) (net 4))
 (segment (start 195.58 96.52) (end 195.58 106.68) (width 1) (layer F.Cu) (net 4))
 (segment (start 195.58 106.68) (end 193.04 109.22) (width 1) (layer F.Cu) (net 4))
 (segment (start 171.2 153.67) (end 173.49 153.67) (width 1) (layer B.Cu) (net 4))
 (segment (start 153.945001 108.925) (end 153.965 108.925) (width 1) (layer F.Cu) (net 4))
 (segment (start 154.94 129.54) (end 152.4 127) (width 1) (layer B.Cu) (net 4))
 (segment (start 151.13 111.740001) (end 153.945001 108.925) (width 1) (layer B.Cu) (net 4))
 (segment (start 151.13 125.73) (end 151.13 111.740001) (width 1) (layer B.Cu) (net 4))
 (segment (start 152.4 127) (end 151.13 125.73) (width 1) (layer B.Cu) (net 4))
 (segment (start 160.02 135.89) (end 160.02 134.62) (width 1) (layer B.Cu) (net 4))
 (segment (start 160.02 134.62) (end 154.94 129.54) (width 1) (layer B.Cu) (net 4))
 (segment (start 169.41 96.52) (end 171.7 96.52) (width 1) (layer B.Cu) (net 4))
 (segment (start 162.56 143.51) (end 162.56 140.97) (width 0.65) (layer B.Cu) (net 10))
 (segment (start 162.56 140.97) (end 160.02 138.43) (width 0.65) (layer B.Cu) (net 10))
 (segment (start 160.02 138.43) (end 156.21 138.43) (width 0.65) (layer B.Cu) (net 10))
 (segment (start 156.21 138.43) (end 152.4 134.62) (width 0.65) (layer B.Cu) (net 10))
 (segment (start 152.4 134.62) (end 152.4 129.54) (width 0.65) (layer B.Cu) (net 10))
 (segment (start 152.4 129.54) (end 149.86 127) (width 0.65) (layer B.Cu) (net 10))
 (segment (start 149.86 127) (end 149.86 109.22) (width 0.65) (layer B.Cu) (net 10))
 (segment (start 149.86 109.22) (end 153.67 105.41) (width 0.65) (layer B.Cu) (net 10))
 (segment (start 153.67 105.41) (end 167.64 105.41) (width 0.65) (layer B.Cu) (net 10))
 (segment (start 167.64 105.41) (end 169.41 103.64) (width 0.65) (layer B.Cu) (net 10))
 (segment (start 169.41 103.64) (end 169.41 101.6) (width 0.65) (layer B.Cu) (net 10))
 (segment (start 175.78 148.59) (end 175.78 147.84) (width 0.65) (layer B.Cu) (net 10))
 (segment (start 175.78 147.84) (end 173.99 146.05) (width 0.65) (layer B.Cu) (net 10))
 (segment (start 173.99 146.05) (end 165.1 146.05) (width 0.65) (layer B.Cu) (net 10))
 (segment (start 165.1 146.05) (end 162.56 143.51) (width 0.65) (layer B.Cu) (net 10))
 (segment (start 160.02 143.51) (end 160.02 140.97) (width 0.65) (layer B.Cu) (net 9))
 (segment (start 165.85 102.87) (end 167.12 101.6) (width 0.65) (layer B.Cu) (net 9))
 (segment (start 152.4 102.87) (end 165.85 102.87) (width 0.65) (layer B.Cu) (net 9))
 (segment (start 148.59 106.68) (end 152.4 102.87) (width 0.65) (layer B.Cu) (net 9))
 (segment (start 148.59 127) (end 148.59 106.68) (width 0.65) (layer B.Cu) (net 9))
 (segment (start 151.13 129.54) (end 148.59 127) (width 0.65) (layer B.Cu) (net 9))
 (segment (start 151.13 135.89) (end 151.13 129.54) (width 0.65) (layer B.Cu) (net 9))
 (segment (start 154.94 139.7) (end 151.13 135.89) (width 0.65) (layer B.Cu) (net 9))
 (segment (start 158.75 139.7) (end 154.94 139.7) (width 0.65) (layer B.Cu) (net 9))
 (segment (start 160.02 140.97) (end 158.75 139.7) (width 0.65) (layer B.Cu) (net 9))
 (segment (start 173.49 148.59) (end 173.49 148.09) (width 0.65) (layer B.Cu) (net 9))
 (segment (start 173.49 148.09) (end 172.300002 146.900002) (width 0.65) (layer B.Cu) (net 9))
 (segment (start 163.410002 146.900002) (end 160.02 143.51) (width 0.65) (layer B.Cu) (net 9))
 (segment (start 172.300002 146.900002) (end 163.410002 146.900002) (width 0.65) (layer B.Cu) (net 9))
 (segment (start 193.04 111.76) (end 191.77 111.76) (width 0.65) (layer B.Cu) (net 18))
 (segment (start 189.23 121.900001) (end 186.965001 124.165) (width 0.65) (layer B.Cu) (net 18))
 (segment (start 189.23 114.3) (end 189.23 121.900001) (width 0.65) (layer B.Cu) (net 18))
 (segment (start 191.77 111.76) (end 189.23 114.3) (width 0.65) (layer B.Cu) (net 18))
 (segment (start 160.02 128.27) (end 160.02 129.54) (width 0.65) (layer B.Cu) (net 20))
 (segment (start 156.485001 124.165) (end 156.485001 124.735001) (width 0.65) (layer B.Cu) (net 20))
 (segment (start 156.485001 124.735001) (end 160.02 128.27) (width 0.65) (layer B.Cu) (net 20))
 (segment (start 162.56 128.27) (end 162.56 129.54) (width 0.65) (layer B.Cu) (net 19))
 (segment (start 159.025001 124.165) (end 159.025001 124.735001) (width 0.65) (layer B.Cu) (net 19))
 (segment (start 159.025001 124.735001) (end 162.56 128.27) (width 0.65) (layer B.Cu) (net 19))
 (segment (start 174.265001 108.925) (end 174.265001 107.674999) (width 0.65) (layer B.Cu) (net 21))
 (segment (start 193.04 105.41) (end 193.04 102.87) (width 0.65) (layer B.Cu) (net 21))
 (segment (start 191.77 106.68) (end 193.04 105.41) (width 0.65) (layer B.Cu) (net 21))
 (segment (start 175.26 106.68) (end 191.77 106.68) (width 0.65) (layer B.Cu) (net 21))
 (segment (start 174.265001 107.674999) (end 175.26 106.68) (width 0.65) (layer B.Cu) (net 21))
 (segment (start 174.265001 108.925) (end 174.285 108.925) (width 0.65) (layer F.Cu) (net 21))
 (segment (start 171.725001 108.925) (end 171.725001 107.674999) (width 0.65) (layer B.Cu) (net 22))
 (segment (start 191.77 100.33) (end 193.04 100.33) (width 0.65) (layer B.Cu) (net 22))
 (segment (start 190.5 101.6) (end 191.77 100.33) (width 0.65) (layer B.Cu) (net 22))
 (segment (start 190.5 102.87) (end 190.5 101.6) (width 0.65) (layer B.Cu) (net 22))
 (segment (start 187.96 105.41) (end 190.5 102.87) (width 0.65) (layer B.Cu) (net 22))
 (segment (start 173.99 105.41) (end 187.96 105.41) (width 0.65) (layer B.Cu) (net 22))
 (segment (start 171.725001 107.674999) (end 173.99 105.41) (width 0.65) (layer B.Cu) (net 22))
 (segment (start 171.725001 108.925) (end 171.745 108.925) (width 0.65) (layer F.Cu) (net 22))
 (segment (start 165.1 135.89) (end 165.1 127) (width 0.65) (layer B.Cu) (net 23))
 (segment (start 164.105001 126.005001) (end 164.105001 124.165) (width 0.65) (layer B.Cu) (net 23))
 (segment (start 165.1 127) (end 164.105001 126.005001) (width 0.65) (layer B.Cu) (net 23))
 (segment (start 157.48 135.89) (end 157.48 134.62) (width 0.65) (layer F.Cu) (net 25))
 (segment (start 166.645001 130.534999) (end 166.645001 124.165) (width 0.65) (layer F.Cu) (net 25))
 (segment (start 163.83 133.35) (end 166.645001 130.534999) (width 0.65) (layer F.Cu) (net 25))
 (segment (start 158.75 133.35) (end 163.83 133.35) (width 0.65) (layer F.Cu) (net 25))
 (segment (start 157.48 134.62) (end 158.75 133.35) (width 0.65) (layer F.Cu) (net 25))
 (segment (start 179.345001 124.165) (end 179.345001 125.454999) (width 0.65) (layer B.Cu) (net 48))
 (segment (start 172.72 132.08) (end 171.45 132.08) (width 0.65) (layer B.Cu) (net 48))
 (segment (start 179.345001 125.454999) (end 172.72 132.08) (width 0.65) (layer B.Cu) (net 48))
 (segment (start 171.725001 124.165) (end 171.725001 127.994999) (width 0.65) (layer F.Cu) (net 51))
 (segment (start 168.91 137.16) (end 171.45 139.7) (width 0.65) (layer F.Cu) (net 51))
 (segment (start 168.91 130.81) (end 168.91 137.16) (width 0.65) (layer F.Cu) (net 51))
 (segment (start 171.725001 127.994999) (end 168.91 130.81) (width 0.65) (layer F.Cu) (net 51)))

